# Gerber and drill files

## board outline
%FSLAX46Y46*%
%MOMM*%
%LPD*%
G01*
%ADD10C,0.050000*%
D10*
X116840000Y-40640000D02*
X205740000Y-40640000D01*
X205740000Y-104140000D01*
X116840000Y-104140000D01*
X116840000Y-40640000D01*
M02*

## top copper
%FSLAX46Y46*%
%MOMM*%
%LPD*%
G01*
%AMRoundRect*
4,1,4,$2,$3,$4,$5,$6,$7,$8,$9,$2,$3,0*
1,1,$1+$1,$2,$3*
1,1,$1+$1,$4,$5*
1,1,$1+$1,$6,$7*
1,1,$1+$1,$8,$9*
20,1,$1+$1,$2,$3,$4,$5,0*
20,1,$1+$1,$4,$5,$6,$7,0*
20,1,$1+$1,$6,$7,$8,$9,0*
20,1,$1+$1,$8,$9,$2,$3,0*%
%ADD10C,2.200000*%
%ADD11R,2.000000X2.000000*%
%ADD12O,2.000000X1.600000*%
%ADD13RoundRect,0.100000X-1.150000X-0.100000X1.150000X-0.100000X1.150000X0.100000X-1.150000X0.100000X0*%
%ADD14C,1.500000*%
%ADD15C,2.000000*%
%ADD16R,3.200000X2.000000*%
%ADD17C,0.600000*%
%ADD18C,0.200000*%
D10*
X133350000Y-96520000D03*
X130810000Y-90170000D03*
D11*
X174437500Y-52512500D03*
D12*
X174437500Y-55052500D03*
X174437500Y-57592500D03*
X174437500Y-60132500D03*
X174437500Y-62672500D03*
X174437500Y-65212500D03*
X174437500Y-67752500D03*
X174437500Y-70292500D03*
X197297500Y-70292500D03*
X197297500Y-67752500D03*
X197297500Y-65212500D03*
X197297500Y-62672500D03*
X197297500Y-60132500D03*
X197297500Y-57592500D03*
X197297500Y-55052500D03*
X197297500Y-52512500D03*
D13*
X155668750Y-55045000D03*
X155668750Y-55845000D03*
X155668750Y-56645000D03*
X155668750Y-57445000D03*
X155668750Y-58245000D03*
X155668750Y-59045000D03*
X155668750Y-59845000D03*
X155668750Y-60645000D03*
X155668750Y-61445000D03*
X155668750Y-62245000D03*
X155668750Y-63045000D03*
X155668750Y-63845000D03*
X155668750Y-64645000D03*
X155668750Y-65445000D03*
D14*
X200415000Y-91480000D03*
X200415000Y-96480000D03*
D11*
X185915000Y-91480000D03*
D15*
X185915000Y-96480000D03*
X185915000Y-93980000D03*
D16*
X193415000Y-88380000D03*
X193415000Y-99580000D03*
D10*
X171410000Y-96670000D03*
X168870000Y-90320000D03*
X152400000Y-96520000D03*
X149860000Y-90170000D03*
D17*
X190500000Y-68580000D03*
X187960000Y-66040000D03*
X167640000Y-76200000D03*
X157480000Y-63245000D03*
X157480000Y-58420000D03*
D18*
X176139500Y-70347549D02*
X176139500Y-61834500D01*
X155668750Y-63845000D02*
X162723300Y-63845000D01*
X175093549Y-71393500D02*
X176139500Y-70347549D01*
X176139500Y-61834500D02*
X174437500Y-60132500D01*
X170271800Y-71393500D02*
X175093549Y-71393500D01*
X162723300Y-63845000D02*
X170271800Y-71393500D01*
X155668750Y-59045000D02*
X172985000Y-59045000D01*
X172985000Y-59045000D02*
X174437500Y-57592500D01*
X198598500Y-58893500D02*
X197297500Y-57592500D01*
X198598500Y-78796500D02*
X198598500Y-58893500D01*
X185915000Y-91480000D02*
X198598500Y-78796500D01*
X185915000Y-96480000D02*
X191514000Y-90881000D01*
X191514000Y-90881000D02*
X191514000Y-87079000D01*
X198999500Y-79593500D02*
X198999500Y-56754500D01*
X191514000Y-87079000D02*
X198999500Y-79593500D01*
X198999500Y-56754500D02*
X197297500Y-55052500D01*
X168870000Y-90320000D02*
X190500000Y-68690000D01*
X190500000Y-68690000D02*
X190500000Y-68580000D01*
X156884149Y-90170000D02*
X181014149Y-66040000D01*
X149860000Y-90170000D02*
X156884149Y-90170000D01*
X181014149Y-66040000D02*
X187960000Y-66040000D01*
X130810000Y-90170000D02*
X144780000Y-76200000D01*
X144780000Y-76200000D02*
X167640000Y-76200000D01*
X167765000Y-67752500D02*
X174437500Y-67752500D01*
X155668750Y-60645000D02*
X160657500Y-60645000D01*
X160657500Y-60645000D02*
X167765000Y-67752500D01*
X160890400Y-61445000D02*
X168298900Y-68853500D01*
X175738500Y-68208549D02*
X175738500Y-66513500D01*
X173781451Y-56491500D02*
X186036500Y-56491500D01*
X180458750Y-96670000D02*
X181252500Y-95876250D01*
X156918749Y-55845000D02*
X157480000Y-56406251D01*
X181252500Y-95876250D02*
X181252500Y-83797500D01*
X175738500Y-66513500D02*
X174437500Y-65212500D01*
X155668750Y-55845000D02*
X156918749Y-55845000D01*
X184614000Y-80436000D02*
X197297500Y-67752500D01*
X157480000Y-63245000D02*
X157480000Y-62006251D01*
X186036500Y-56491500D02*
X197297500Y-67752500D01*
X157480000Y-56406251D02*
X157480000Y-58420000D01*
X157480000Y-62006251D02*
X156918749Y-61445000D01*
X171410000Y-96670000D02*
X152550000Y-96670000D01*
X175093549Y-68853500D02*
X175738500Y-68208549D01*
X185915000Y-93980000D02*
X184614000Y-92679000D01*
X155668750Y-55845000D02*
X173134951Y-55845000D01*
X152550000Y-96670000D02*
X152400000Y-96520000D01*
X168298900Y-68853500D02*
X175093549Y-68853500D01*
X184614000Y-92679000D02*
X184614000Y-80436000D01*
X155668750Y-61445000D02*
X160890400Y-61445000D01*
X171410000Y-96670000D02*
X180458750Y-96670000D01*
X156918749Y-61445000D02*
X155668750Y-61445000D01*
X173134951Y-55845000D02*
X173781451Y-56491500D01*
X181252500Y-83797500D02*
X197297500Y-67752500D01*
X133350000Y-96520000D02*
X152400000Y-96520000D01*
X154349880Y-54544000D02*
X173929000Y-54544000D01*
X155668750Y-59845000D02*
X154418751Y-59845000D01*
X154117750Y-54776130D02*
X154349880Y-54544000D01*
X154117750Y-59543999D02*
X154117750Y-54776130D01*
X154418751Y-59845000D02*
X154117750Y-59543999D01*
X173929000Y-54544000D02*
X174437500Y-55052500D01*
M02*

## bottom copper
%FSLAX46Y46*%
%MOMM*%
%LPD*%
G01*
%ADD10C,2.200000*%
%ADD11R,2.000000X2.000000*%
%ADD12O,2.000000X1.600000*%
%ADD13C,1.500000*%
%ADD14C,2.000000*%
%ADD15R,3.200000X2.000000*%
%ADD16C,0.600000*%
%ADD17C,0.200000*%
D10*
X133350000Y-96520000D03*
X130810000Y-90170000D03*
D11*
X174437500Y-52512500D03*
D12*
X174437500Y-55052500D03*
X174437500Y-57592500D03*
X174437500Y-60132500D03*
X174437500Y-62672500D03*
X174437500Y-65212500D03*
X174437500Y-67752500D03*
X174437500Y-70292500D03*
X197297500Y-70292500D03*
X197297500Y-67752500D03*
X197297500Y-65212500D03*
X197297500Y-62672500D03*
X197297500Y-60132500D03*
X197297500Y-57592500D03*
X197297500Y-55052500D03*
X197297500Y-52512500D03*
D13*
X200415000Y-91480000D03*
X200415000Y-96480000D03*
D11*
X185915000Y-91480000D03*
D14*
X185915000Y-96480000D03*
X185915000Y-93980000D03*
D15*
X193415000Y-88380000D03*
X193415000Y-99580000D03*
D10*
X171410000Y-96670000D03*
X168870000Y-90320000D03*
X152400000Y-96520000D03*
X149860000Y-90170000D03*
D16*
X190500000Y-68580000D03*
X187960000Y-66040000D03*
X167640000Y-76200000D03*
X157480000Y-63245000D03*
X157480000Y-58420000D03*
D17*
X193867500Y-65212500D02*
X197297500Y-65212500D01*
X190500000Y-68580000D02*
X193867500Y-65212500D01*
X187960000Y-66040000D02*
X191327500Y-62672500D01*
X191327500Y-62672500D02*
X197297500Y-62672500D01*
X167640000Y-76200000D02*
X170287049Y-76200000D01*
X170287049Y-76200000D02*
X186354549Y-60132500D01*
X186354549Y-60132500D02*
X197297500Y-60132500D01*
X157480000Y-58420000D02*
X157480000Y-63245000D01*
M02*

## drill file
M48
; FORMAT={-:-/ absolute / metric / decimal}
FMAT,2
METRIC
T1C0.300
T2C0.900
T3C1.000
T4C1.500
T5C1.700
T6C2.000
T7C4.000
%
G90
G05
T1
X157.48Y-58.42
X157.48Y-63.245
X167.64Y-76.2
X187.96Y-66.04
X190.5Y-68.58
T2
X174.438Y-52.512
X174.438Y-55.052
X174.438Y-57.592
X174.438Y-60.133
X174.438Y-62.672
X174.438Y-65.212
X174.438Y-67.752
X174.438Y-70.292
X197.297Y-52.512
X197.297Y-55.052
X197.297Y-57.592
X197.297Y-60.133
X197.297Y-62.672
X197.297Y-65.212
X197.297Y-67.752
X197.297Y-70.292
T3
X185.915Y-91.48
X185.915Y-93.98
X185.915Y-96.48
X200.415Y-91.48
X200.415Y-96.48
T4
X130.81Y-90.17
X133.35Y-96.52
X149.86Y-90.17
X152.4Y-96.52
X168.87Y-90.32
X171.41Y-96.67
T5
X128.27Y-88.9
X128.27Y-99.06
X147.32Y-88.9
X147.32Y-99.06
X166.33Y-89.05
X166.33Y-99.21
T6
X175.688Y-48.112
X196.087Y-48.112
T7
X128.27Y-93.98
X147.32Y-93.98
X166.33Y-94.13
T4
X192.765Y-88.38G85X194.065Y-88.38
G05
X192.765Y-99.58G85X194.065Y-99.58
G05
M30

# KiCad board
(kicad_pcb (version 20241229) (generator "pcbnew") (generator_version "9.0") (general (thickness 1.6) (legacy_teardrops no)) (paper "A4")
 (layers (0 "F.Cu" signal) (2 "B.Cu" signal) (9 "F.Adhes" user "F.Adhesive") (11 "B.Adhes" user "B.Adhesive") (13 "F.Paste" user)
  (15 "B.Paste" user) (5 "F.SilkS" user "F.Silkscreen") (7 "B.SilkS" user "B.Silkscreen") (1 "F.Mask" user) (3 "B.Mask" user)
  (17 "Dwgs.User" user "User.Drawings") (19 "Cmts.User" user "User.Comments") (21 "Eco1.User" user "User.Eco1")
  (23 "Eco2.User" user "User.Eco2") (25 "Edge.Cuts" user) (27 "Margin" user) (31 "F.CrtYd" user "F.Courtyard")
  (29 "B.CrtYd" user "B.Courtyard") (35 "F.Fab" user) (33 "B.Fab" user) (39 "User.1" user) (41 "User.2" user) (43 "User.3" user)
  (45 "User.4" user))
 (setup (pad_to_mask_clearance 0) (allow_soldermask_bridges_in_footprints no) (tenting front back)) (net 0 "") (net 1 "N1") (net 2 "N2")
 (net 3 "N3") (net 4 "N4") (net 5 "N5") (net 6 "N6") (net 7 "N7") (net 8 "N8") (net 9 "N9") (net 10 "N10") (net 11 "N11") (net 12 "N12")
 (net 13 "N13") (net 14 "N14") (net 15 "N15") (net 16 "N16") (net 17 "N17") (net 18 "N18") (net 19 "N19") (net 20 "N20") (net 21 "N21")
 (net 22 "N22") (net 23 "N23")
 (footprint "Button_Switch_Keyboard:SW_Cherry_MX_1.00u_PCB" (layer "F.Cu") (at 133.35 96.52 -90)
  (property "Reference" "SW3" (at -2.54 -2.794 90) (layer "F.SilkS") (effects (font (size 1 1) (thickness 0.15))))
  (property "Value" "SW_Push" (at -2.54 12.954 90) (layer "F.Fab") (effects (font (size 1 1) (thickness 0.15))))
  (pad "" np_thru_hole circle (at -7.62 5.08 270) (size 1.7 1.7) (drill 1.7) (layers "*.Cu" "*.Mask"))
  (pad "" np_thru_hole circle (at -2.54 5.08 270) (size 4 4) (drill 4) (layers "*.Cu" "*.Mask"))
  (pad "" np_thru_hole circle (at 2.54 5.08 270) (size 1.7 1.7) (drill 1.7) (layers "*.Cu" "*.Mask"))
  (pad "1" thru_hole circle (at 0 0 270) (size 2.2 2.2) (drill 1.5) (layers "*.Cu" "*.Mask") (remove_unused_layers no) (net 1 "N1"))
  (pad "2" thru_hole circle (at -6.35 2.54 270) (size 2.2 2.2) (drill 1.5) (layers "*.Cu" "*.Mask") (remove_unused_layers no) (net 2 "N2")))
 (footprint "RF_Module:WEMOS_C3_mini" (layer "F.Cu") (at 174.4375 52.5125)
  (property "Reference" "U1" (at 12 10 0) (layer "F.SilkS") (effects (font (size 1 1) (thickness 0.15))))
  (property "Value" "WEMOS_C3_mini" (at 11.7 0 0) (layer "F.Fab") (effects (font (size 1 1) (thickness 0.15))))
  (pad "" np_thru_hole circle (at 1.25 -4.4) (size 3 3) (drill 2) (layers "*.Mask"))
  (pad "" np_thru_hole circle (at 21.65 -4.4) (size 3 3) (drill 2) (layers "*.Mask"))
  (pad "1" thru_hole rect (at 0 0) (size 2 2) (drill 0.9) (layers "*.Cu" "*.Mask") (remove_unused_layers no) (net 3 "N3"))
  (pad "2" thru_hole oval (at 0 2.54) (size 2 1.6) (drill 0.9) (layers "*.Cu" "*.Mask") (remove_unused_layers no) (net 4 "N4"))
  (pad "3" thru_hole oval (at 0 5.08) (size 2 1.6) (drill 0.9) (layers "*.Cu" "*.Mask") (remove_unused_layers no) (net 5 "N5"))
  (pad "4" thru_hole oval (at 0 7.62) (size 2 1.6) (drill 0.9) (layers "*.Cu" "*.Mask") (remove_unused_layers no) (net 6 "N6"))
  (pad "5" thru_hole oval (at 0 10.16) (size 2 1.6) (drill 0.9) (layers "*.Cu" "*.Mask") (remove_unused_layers no) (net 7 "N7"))
  (pad "6" thru_hole oval (at 0 12.7) (size 2 1.6) (drill 0.9) (layers "*.Cu" "*.Mask") (remove_unused_layers no) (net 1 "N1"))
  (pad "7" thru_hole oval (at 0 15.24) (size 2 1.6) (drill 0.9) (layers "*.Cu" "*.Mask") (remove_unused_layers no) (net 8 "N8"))
  (pad "8" thru_hole oval (at 0 17.78) (size 2 1.6) (drill 0.9) (layers "*.Cu" "*.Mask") (remove_unused_layers no) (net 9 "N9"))
  (pad "9" thru_hole oval (at 22.86 17.78) (size 2 1.6) (drill 0.9) (layers "*.Cu" "*.Mask") (remove_unused_layers no) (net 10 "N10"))
  (pad "10" thru_hole oval (at 22.86 15.24) (size 2 1.6) (drill 0.9) (layers "*.Cu" "*.Mask") (remove_unused_layers no) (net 1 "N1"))
  (pad "11" thru_hole oval (at 22.86 12.7) (size 2 1.6) (drill 0.9) (layers "*.Cu" "*.Mask") (remove_unused_layers no) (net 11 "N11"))
  (pad "12" thru_hole oval (at 22.86 10.16) (size 2 1.6) (drill 0.9) (layers "*.Cu" "*.Mask") (remove_unused_layers no) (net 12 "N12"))
  (pad "13" thru_hole oval (at 22.86 7.62) (size 2 1.6) (drill 0.9) (layers "*.Cu" "*.Mask") (remove_unused_layers no) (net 2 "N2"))
  (pad "14" thru_hole oval (at 22.86 5.08) (size 2 1.6) (drill 0.9) (layers "*.Cu" "*.Mask") (remove_unused_layers no) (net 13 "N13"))
  (pad "15" thru_hole oval (at 22.86 2.54) (size 2 1.6) (drill 0.9) (layers "*.Cu" "*.Mask") (remove_unused_layers no) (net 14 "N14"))
  (pad "16" thru_hole oval (at 22.86 0) (size 2 1.6) (drill 0.9) (layers "*.Cu" "*.Mask") (remove_unused_layers no) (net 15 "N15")))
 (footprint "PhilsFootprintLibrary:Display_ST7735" (layer "F.Cu") (at 119.26875 43.245)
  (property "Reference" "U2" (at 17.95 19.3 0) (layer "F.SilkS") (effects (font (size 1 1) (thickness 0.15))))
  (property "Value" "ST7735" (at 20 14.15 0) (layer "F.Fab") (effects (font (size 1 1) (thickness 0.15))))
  (pad "1" smd roundrect (at 36.4 11.8) (size 2.5 0.4) (layers "F.Cu" "F.Mask" "F.Paste") (roundrect_rratio 0.25) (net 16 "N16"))
  (pad "2" smd roundrect (at 36.4 12.6) (size 2.5 0.4) (layers "F.Cu" "F.Mask" "F.Paste") (roundrect_rratio 0.25) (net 1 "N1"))
  (pad "3" smd roundrect (at 36.4 13.4) (size 2.5 0.4) (layers "F.Cu" "F.Mask" "F.Paste") (roundrect_rratio 0.25) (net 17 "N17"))
  (pad "4" smd roundrect (at 36.4 14.2) (size 2.5 0.4) (layers "F.Cu" "F.Mask" "F.Paste") (roundrect_rratio 0.25) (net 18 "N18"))
  (pad "5" smd roundrect (at 36.4 15) (size 2.5 0.4) (layers "F.Cu" "F.Mask" "F.Paste") (roundrect_rratio 0.25) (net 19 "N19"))
  (pad "6" smd roundrect (at 36.4 15.8) (size 2.5 0.4) (layers "F.Cu" "F.Mask" "F.Paste") (roundrect_rratio 0.25) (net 5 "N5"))
  (pad "7" smd roundrect (at 36.4 16.6) (size 2.5 0.4) (layers "F.Cu" "F.Mask" "F.Paste") (roundrect_rratio 0.25) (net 4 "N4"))
  (pad "8" smd roundrect (at 36.4 17.4) (size 2.5 0.4) (layers "F.Cu" "F.Mask" "F.Paste") (roundrect_rratio 0.25) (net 8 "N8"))
  (pad "9" smd roundrect (at 36.4 18.2) (size 2.5 0.4) (layers "F.Cu" "F.Mask" "F.Paste") (roundrect_rratio 0.25) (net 1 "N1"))
  (pad "10" smd roundrect (at 36.4 19) (size 2.5 0.4) (layers "F.Cu" "F.Mask" "F.Paste") (roundrect_rratio 0.25) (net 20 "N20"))
  (pad "11" smd roundrect (at 36.4 19.8) (size 2.5 0.4) (layers "F.Cu" "F.Mask" "F.Paste") (roundrect_rratio 0.25) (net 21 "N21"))
  (pad "12" smd roundrect (at 36.4 20.6) (size 2.5 0.4) (layers "F.Cu" "F.Mask" "F.Paste") (roundrect_rratio 0.25) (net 6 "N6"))
  (pad "13" smd roundrect (at 36.4 21.4) (size 2.5 0.4) (layers "F.Cu" "F.Mask" "F.Paste") (roundrect_rratio 0.25) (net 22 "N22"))
  (pad "14" smd roundrect (at 36.4 22.2) (size 2.5 0.4) (layers "F.Cu" "F.Mask" "F.Paste") (roundrect_rratio 0.25) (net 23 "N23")))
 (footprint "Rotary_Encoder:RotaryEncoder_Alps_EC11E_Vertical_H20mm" (layer "F.Cu") (at 185.915 91.48)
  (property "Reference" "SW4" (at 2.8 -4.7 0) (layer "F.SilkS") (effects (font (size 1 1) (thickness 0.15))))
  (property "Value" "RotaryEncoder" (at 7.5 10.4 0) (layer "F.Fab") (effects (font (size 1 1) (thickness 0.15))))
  (pad "" thru_hole circle (at 14.5 0) (size 1.5 1.5) (drill 1) (layers "*.Cu" "*.Mask") (remove_unused_layers no))
  (pad "" thru_hole circle (at 14.5 5) (size 1.5 1.5) (drill 1) (layers "*.Cu" "*.Mask") (remove_unused_layers no))
  (pad "A" thru_hole rect (at 0 0) (size 2 2) (drill 1) (layers "*.Cu" "*.Mask") (remove_unused_layers no) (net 13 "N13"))
  (pad "B" thru_hole circle (at 0 5) (size 2 2) (drill 1) (layers "*.Cu" "*.Mask") (remove_unused_layers no) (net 14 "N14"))
  (pad "C" thru_hole circle (at 0 2.5) (size 2 2) (drill 1) (layers "*.Cu" "*.Mask") (remove_unused_layers no) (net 1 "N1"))
  (pad "MP" thru_hole rect (at 7.5 -3.1) (size 3.2 2) (drill oval 2.8 1.5) (layers "*.Cu" "*.Mask") (remove_unused_layers no))
  (pad "MP" thru_hole rect (at 7.5 8.1) (size 3.2 2) (drill oval 2.8 1.5) (layers "*.Cu" "*.Mask") (remove_unused_layers no)))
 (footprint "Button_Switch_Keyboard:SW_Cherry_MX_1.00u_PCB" (layer "F.Cu") (at 171.41 96.67 -90)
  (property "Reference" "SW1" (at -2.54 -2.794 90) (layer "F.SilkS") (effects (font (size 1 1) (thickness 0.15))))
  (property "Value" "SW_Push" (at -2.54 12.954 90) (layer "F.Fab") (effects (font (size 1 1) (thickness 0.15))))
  (pad "" np_thru_hole circle (at -7.62 5.08 270) (size 1.7 1.7) (drill 1.7) (layers "*.Cu" "*.Mask"))
  (pad "" np_thru_hole circle (at -2.54 5.08 270) (size 4 4) (drill 4) (layers "*.Cu" "*.Mask"))
  (pad "" np_thru_hole circle (at 2.54 5.08 270) (size 1.7 1.7) (drill 1.7) (layers "*.Cu" "*.Mask"))
  (pad "1" thru_hole circle (at 0 0 270) (size 2.2 2.2) (drill 1.5) (layers "*.Cu" "*.Mask") (remove_unused_layers no) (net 1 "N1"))
  (pad "2" thru_hole circle (at -6.35 2.54 270) (size 2.2 2.2) (drill 1.5) (layers "*.Cu" "*.Mask") (remove_unused_layers no) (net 11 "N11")))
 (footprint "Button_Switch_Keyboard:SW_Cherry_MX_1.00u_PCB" (layer "F.Cu") (at 152.4 96.52 -90)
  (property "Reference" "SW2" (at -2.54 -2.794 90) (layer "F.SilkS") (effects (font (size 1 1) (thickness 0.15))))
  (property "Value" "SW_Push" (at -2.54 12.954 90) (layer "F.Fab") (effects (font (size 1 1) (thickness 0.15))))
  (pad "" np_thru_hole circle (at -7.62 5.08 270) (size 1.7 1.7) (drill 1.7) (layers "*.Cu" "*.Mask"))
  (pad "" np_thru_hole circle (at -2.54 5.08 270) (size 4 4) (drill 4) (layers "*.Cu" "*.Mask"))
  (pad "" np_thru_hole circle (at 2.54 5.08 270) (size 1.7 1.7) (drill 1.7) (layers "*.Cu" "*.Mask"))
  (pad "1" thru_hole circle (at 0 0 270) (size 2.2 2.2) (drill 1.5) (layers "*.Cu" "*.Mask") (remove_unused_layers no) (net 1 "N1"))
  (pad "2" thru_hole circle (at -6.35 2.54 270) (size 2.2 2.2) (drill 1.5) (layers "*.Cu" "*.Mask") (remove_unused_layers no) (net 12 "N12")))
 (gr_rect (start 116.84 40.64) (end 205.74 104.14) (stroke (width 0.05) (type default)) (fill no) (layer "Edge.Cuts"))
 (segment (start 176.1395 70.347549) (end 176.1395 61.8345) (width 0.2) (layer "F.Cu") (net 6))
 (segment (start 155.66875 63.845) (end 162.7233 63.845) (width 0.2) (layer "F.Cu") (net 6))
 (segment (start 175.093549 71.3935) (end 176.1395 70.347549) (width 0.2) (layer "F.Cu") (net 6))
 (segment (start 176.1395 61.8345) (end 174.4375 60.1325) (width 0.2) (layer "F.Cu") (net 6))
 (segment (start 170.2718 71.3935) (end 175.093549 71.3935) (width 0.2) (layer "F.Cu") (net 6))
 (segment (start 162.7233 63.845) (end 170.2718 71.3935) (width 0.2) (layer "F.Cu") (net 6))
 (segment (start 155.66875 59.045) (end 172.985 59.045) (width 0.2) (layer "F.Cu") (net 5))
 (segment (start 172.985 59.045) (end 174.4375 57.5925) (width 0.2) (layer "F.Cu") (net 5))
 (segment (start 198.5985 58.8935) (end 197.2975 57.5925) (width 0.2) (layer "F.Cu") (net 13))
 (segment (start 198.5985 78.7965) (end 198.5985 58.8935) (width 0.2) (layer "F.Cu") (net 13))
 (segment (start 185.915 91.48) (end 198.5985 78.7965) (width 0.2) (layer "F.Cu") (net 13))
 (segment (start 185.915 96.48) (end 191.514 90.881) (width 0.2) (layer "F.Cu") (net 14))
 (segment (start 191.514 90.881) (end 191.514 87.079) (width 0.2) (layer "F.Cu") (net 14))
 (segment (start 198.9995 79.5935) (end 198.9995 56.7545) (width 0.2) (layer "F.Cu") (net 14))
 (segment (start 191.514 87.079) (end 198.9995 79.5935) (width 0.2) (layer "F.Cu") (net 14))
 (segment (start 198.9995 56.7545) (end 197.2975 55.0525) (width 0.2) (layer "F.Cu") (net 14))
 (segment (start 168.87 90.32) (end 190.5 68.69) (width 0.2) (layer "F.Cu") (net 11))
 (segment (start 190.5 68.69) (end 190.5 68.58) (width 0.2) (layer "F.Cu") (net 11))
 (via (at 190.5 68.58) (size 0.6) (drill 0.3) (layers "F.Cu" "B.Cu") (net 11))
 (segment (start 193.8675 65.2125) (end 197.2975 65.2125) (width 0.2) (layer "B.Cu") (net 11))
 (segment (start 190.5 68.58) (end 193.8675 65.2125) (width 0.2) (layer "B.Cu") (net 11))
 (segment (start 156.884149 90.17) (end 181.014149 66.04) (width 0.2) (layer "F.Cu") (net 12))
 (segment (start 149.86 90.17) (end 156.884149 90.17) (width 0.2) (layer "F.Cu") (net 12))
 (segment (start 181.014149 66.04) (end 187.96 66.04) (width 0.2) (layer "F.Cu") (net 12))
 (via (at 187.96 66.04) (size 0.6) (drill 0.3) (layers "F.Cu" "B.Cu") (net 12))
 (segment (start 187.96 66.04) (end 191.3275 62.6725) (width 0.2) (layer "B.Cu") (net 12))
 (segment (start 191.3275 62.6725) (end 197.2975 62.6725) (width 0.2) (layer "B.Cu") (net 12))
 (segment (start 130.81 90.17) (end 144.78 76.2) (width 0.2) (layer "F.Cu") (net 2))
 (segment (start 144.78 76.2) (end 167.64 76.2) (width 0.2) (layer "F.Cu") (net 2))
 (via (at 167.64 76.2) (size 0.6) (drill 0.3) (layers "F.Cu" "B.Cu") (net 2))
 (segment (start 167.64 76.2) (end 170.287049 76.2) (width 0.2) (layer "B.Cu") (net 2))
 (segment (start 170.287049 76.2) (end 186.354549 60.1325) (width 0.2) (layer "B.Cu") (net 2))
 (segment (start 186.354549 60.1325) (end 197.2975 60.1325) (width 0.2) (layer "B.Cu") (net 2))
 (segment (start 167.765 67.7525) (end 174.4375 67.7525) (width 0.2) (layer "F.Cu") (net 8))
 (segment (start 155.66875 60.645) (end 160.6575 60.645) (width 0.2) (layer "F.Cu") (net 8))
 (segment (start 160.6575 60.645) (end 167.765 67.7525) (width 0.2) (layer "F.Cu") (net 8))
 (segment (start 160.8904 61.445) (end 168.2989 68.8535) (width 0.2) (layer "F.Cu") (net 1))
 (segment (start 175.7385 68.208549) (end 175.7385 66.5135) (width 0.2) (layer "F.Cu") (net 1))
 (segment (start 173.781451 56.4915) (end 186.0365 56.4915) (width 0.2) (layer "F.Cu") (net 1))
 (segment (start 180.45875 96.67) (end 181.2525 95.87625) (width 0.2) (layer "F.Cu") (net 1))
 (segment (start 156.918749 55.845) (end 157.48 56.406251) (width 0.2) (layer "F.Cu") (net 1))
 (segment (start 181.2525 95.87625) (end 181.2525 83.7975) (width 0.2) (layer "F.Cu") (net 1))
 (segment (start 175.7385 66.5135) (end 174.4375 65.2125) (width 0.2) (layer "F.Cu") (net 1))
 (segment (start 155.66875 55.845) (end 156.918749 55.845) (width 0.2) (layer "F.Cu") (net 1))
 (segment (start 184.614 80.436) (end 197.2975 67.7525) (width 0.2) (layer "F.Cu") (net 1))
 (segment (start 157.48 63.245) (end 157.48 62.006251) (width 0.2) (layer "F.Cu") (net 1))
 (segment (start 186.0365 56.4915) (end 197.2975 67.7525) (width 0.2) (layer "F.Cu") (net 1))
 (segment (start 157.48 56.406251) (end 157.48 58.42) (width 0.2) (layer "F.Cu") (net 1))
 (segment (start 157.48 62.006251) (end 156.918749 61.445) (width 0.2) (layer "F.Cu") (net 1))
 (segment (start 171.41 96.67) (end 152.55 96.67) (width 0.2) (layer "F.Cu") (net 1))
 (segment (start 175.093549 68.8535) (end 175.7385 68.208549) (width 0.2) (layer "F.Cu") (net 1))
 (segment (start 185.915 93.98) (end 184.614 92.679) (width 0.2) (layer "F.Cu") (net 1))
 (segment (start 155.66875 55.845) (end 173.134951 55.845) (width 0.2) (layer "F.Cu") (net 1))
 (segment (start 152.55 96.67) (end 152.4 96.52) (width 0.2) (layer "F.Cu") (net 1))
 (segment (start 168.2989 68.8535) (end 175.093549 68.8535) (width 0.2) (layer "F.Cu") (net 1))
 (segment (start 184.614 92.679) (end 184.614 80.436) (width 0.2) (layer "F.Cu") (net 1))
 (segment (start 155.66875 61.445) (end 160.8904 61.445) (width 0.2) (layer "F.Cu") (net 1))
 (segment (start 171.41 96.67) (end 180.45875 96.67) (width 0.2) (layer "F.Cu") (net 1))
 (segment (start 156.918749 61.445) (end 155.66875 61.445) (width 0.2) (layer "F.Cu") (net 1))
 (segment (start 173.134951 55.845) (end 173.781451 56.4915) (width 0.2) (layer "F.Cu") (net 1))
 (segment (start 181.2525 83.7975) (end 197.2975 67.7525) (width 0.2) (layer "F.Cu") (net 1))
 (segment (start 133.35 96.52) (end 152.4 96.52) (width 0.2) (layer "F.Cu") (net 1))
 (via (at 157.48 63.245) (size 0.6) (drill 0.3) (layers "F.Cu" "B.Cu") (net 1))
 (via (at 157.48 58.42) (size 0.6) (drill 0.3) (layers "F.Cu" "B.Cu") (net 1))
 (segment (start 157.48 58.42) (end 157.48 63.245) (width 0.2) (layer "B.Cu") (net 1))
 (segment (start 154.34988 54.544) (end 173.929 54.544) (width 0.2) (layer "F.Cu") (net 4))
 (segment (start 155.66875 59.845) (end 154.418751 59.845) (width 0.2) (layer "F.Cu") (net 4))
 (segment (start 154.11775 54.77613) (end 154.34988 54.544) (width 0.2) (layer "F.Cu") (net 4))
 (segment (start 154.11775 59.543999) (end 154.11775 54.77613) (width 0.2) (layer "F.Cu") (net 4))
 (segment (start 154.418751 59.845) (end 154.11775 59.543999) (width 0.2) (layer "F.Cu") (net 4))
 (segment (start 173.929 54.544) (end 174.4375 55.0525) (width 0.2) (layer "F.Cu") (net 4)))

